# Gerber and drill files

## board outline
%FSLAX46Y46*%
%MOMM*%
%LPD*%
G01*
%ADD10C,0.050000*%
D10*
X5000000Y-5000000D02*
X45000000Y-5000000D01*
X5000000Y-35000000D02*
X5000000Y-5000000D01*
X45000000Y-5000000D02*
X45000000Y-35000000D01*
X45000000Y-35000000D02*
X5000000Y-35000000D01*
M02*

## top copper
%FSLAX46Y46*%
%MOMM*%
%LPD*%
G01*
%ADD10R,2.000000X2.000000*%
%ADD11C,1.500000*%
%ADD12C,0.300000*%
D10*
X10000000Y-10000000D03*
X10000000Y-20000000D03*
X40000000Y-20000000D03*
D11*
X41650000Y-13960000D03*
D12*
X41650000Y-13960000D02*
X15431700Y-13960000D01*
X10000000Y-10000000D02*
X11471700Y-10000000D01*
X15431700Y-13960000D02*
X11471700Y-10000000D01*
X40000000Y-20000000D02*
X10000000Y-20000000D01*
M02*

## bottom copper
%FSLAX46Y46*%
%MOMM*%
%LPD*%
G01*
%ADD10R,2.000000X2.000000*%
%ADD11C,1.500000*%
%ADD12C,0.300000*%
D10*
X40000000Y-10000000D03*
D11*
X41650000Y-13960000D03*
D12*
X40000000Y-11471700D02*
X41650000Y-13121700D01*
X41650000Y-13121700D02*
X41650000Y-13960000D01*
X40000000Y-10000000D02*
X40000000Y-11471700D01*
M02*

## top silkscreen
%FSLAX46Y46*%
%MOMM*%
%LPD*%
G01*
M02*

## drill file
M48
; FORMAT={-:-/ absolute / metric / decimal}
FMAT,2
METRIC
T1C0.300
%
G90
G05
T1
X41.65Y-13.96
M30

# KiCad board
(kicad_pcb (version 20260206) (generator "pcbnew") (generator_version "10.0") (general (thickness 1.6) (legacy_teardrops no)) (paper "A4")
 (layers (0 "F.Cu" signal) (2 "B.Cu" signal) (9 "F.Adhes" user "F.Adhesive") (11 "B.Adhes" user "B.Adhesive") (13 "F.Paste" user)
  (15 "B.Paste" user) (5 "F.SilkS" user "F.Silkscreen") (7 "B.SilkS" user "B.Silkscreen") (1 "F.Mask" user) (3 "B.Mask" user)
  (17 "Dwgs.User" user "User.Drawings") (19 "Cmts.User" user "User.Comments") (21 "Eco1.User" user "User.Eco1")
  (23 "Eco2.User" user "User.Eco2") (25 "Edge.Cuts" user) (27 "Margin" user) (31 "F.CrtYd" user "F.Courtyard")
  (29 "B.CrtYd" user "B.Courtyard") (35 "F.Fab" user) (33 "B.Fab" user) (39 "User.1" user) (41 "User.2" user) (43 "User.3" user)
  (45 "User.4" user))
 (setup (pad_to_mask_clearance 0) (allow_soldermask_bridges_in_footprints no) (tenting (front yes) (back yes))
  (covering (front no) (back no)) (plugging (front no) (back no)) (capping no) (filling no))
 (gr_line (start 5 5) (end 45 5) (stroke (width 0.05) (type default)) (layer "Edge.Cuts"))
 (gr_line (start 5 35) (end 5 5) (stroke (width 0.05) (type default)) (layer "Edge.Cuts"))
 (gr_line (start 45 5) (end 45 35) (stroke (width 0.05) (type default)) (layer "Edge.Cuts"))
 (gr_line (start 45 35) (end 5 35) (stroke (width 0.05) (type default)) (layer "Edge.Cuts"))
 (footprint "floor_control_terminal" (layer "F.Cu") (at 10 10)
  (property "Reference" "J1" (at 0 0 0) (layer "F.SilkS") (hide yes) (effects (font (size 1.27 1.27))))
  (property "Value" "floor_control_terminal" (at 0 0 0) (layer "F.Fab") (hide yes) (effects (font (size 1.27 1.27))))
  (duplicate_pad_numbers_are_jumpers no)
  (pad "1" smd rect (at 0 0) (size 2 2) (layers "F.Cu" "F.Paste" "F.Mask") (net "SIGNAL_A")))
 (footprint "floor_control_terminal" (layer "B.Cu") (at 40 10)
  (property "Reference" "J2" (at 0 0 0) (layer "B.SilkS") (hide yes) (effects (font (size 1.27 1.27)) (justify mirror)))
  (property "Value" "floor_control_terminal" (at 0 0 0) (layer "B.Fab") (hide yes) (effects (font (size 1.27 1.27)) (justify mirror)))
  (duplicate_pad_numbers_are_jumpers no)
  (pad "1" smd rect (at 0 0) (size 2 2) (layers "B.Cu" "B.Paste" "B.Mask") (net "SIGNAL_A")))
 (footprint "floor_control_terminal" (layer "F.Cu") (at 10 20)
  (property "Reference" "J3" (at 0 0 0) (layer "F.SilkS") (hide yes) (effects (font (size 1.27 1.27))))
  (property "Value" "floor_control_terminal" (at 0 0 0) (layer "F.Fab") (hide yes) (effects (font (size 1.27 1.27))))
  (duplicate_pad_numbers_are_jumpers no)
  (pad "1" smd rect (at 0 0) (size 2 2) (layers "F.Cu" "F.Paste" "F.Mask") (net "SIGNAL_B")))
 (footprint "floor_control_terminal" (layer "F.Cu") (at 40 20)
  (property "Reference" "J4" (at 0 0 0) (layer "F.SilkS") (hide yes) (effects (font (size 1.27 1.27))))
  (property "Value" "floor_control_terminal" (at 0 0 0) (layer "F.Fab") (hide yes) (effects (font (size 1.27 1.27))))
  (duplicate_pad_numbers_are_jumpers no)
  (pad "1" smd rect (at 0 0) (size 2 2) (layers "F.Cu" "F.Paste" "F.Mask") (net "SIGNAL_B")))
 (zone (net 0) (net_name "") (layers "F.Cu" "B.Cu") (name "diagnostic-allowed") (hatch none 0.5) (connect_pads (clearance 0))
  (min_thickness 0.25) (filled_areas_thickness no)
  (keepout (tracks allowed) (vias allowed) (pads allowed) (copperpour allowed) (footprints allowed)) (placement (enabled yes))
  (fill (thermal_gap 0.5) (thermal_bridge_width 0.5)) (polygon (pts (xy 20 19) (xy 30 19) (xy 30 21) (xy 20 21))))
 (segment (start 41.65 13.96) (end 15.4317 13.96) (width 0.3) (layer "F.Cu") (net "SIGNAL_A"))
 (segment (start 10 10) (end 11.4717 10) (width 0.3) (layer "F.Cu") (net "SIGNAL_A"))
 (segment (start 15.4317 13.96) (end 11.4717 10) (width 0.3) (layer "F.Cu") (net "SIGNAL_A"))
 (via (at 41.65 13.96) (size 1.5) (drill 0.3) (layers "F.Cu" "B.Cu") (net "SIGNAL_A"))
 (segment (start 40 11.4717) (end 41.65 13.1217) (width 0.3) (layer "B.Cu") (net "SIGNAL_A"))
 (segment (start 41.65 13.1217) (end 41.65 13.96) (width 0.3) (layer "B.Cu") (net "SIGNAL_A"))
 (segment (start 40 10) (end 40 11.4717) (width 0.3) (layer "B.Cu") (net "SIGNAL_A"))
 (segment (start 40 20) (end 10 20) (width 0.3) (layer "F.Cu") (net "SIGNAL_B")))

